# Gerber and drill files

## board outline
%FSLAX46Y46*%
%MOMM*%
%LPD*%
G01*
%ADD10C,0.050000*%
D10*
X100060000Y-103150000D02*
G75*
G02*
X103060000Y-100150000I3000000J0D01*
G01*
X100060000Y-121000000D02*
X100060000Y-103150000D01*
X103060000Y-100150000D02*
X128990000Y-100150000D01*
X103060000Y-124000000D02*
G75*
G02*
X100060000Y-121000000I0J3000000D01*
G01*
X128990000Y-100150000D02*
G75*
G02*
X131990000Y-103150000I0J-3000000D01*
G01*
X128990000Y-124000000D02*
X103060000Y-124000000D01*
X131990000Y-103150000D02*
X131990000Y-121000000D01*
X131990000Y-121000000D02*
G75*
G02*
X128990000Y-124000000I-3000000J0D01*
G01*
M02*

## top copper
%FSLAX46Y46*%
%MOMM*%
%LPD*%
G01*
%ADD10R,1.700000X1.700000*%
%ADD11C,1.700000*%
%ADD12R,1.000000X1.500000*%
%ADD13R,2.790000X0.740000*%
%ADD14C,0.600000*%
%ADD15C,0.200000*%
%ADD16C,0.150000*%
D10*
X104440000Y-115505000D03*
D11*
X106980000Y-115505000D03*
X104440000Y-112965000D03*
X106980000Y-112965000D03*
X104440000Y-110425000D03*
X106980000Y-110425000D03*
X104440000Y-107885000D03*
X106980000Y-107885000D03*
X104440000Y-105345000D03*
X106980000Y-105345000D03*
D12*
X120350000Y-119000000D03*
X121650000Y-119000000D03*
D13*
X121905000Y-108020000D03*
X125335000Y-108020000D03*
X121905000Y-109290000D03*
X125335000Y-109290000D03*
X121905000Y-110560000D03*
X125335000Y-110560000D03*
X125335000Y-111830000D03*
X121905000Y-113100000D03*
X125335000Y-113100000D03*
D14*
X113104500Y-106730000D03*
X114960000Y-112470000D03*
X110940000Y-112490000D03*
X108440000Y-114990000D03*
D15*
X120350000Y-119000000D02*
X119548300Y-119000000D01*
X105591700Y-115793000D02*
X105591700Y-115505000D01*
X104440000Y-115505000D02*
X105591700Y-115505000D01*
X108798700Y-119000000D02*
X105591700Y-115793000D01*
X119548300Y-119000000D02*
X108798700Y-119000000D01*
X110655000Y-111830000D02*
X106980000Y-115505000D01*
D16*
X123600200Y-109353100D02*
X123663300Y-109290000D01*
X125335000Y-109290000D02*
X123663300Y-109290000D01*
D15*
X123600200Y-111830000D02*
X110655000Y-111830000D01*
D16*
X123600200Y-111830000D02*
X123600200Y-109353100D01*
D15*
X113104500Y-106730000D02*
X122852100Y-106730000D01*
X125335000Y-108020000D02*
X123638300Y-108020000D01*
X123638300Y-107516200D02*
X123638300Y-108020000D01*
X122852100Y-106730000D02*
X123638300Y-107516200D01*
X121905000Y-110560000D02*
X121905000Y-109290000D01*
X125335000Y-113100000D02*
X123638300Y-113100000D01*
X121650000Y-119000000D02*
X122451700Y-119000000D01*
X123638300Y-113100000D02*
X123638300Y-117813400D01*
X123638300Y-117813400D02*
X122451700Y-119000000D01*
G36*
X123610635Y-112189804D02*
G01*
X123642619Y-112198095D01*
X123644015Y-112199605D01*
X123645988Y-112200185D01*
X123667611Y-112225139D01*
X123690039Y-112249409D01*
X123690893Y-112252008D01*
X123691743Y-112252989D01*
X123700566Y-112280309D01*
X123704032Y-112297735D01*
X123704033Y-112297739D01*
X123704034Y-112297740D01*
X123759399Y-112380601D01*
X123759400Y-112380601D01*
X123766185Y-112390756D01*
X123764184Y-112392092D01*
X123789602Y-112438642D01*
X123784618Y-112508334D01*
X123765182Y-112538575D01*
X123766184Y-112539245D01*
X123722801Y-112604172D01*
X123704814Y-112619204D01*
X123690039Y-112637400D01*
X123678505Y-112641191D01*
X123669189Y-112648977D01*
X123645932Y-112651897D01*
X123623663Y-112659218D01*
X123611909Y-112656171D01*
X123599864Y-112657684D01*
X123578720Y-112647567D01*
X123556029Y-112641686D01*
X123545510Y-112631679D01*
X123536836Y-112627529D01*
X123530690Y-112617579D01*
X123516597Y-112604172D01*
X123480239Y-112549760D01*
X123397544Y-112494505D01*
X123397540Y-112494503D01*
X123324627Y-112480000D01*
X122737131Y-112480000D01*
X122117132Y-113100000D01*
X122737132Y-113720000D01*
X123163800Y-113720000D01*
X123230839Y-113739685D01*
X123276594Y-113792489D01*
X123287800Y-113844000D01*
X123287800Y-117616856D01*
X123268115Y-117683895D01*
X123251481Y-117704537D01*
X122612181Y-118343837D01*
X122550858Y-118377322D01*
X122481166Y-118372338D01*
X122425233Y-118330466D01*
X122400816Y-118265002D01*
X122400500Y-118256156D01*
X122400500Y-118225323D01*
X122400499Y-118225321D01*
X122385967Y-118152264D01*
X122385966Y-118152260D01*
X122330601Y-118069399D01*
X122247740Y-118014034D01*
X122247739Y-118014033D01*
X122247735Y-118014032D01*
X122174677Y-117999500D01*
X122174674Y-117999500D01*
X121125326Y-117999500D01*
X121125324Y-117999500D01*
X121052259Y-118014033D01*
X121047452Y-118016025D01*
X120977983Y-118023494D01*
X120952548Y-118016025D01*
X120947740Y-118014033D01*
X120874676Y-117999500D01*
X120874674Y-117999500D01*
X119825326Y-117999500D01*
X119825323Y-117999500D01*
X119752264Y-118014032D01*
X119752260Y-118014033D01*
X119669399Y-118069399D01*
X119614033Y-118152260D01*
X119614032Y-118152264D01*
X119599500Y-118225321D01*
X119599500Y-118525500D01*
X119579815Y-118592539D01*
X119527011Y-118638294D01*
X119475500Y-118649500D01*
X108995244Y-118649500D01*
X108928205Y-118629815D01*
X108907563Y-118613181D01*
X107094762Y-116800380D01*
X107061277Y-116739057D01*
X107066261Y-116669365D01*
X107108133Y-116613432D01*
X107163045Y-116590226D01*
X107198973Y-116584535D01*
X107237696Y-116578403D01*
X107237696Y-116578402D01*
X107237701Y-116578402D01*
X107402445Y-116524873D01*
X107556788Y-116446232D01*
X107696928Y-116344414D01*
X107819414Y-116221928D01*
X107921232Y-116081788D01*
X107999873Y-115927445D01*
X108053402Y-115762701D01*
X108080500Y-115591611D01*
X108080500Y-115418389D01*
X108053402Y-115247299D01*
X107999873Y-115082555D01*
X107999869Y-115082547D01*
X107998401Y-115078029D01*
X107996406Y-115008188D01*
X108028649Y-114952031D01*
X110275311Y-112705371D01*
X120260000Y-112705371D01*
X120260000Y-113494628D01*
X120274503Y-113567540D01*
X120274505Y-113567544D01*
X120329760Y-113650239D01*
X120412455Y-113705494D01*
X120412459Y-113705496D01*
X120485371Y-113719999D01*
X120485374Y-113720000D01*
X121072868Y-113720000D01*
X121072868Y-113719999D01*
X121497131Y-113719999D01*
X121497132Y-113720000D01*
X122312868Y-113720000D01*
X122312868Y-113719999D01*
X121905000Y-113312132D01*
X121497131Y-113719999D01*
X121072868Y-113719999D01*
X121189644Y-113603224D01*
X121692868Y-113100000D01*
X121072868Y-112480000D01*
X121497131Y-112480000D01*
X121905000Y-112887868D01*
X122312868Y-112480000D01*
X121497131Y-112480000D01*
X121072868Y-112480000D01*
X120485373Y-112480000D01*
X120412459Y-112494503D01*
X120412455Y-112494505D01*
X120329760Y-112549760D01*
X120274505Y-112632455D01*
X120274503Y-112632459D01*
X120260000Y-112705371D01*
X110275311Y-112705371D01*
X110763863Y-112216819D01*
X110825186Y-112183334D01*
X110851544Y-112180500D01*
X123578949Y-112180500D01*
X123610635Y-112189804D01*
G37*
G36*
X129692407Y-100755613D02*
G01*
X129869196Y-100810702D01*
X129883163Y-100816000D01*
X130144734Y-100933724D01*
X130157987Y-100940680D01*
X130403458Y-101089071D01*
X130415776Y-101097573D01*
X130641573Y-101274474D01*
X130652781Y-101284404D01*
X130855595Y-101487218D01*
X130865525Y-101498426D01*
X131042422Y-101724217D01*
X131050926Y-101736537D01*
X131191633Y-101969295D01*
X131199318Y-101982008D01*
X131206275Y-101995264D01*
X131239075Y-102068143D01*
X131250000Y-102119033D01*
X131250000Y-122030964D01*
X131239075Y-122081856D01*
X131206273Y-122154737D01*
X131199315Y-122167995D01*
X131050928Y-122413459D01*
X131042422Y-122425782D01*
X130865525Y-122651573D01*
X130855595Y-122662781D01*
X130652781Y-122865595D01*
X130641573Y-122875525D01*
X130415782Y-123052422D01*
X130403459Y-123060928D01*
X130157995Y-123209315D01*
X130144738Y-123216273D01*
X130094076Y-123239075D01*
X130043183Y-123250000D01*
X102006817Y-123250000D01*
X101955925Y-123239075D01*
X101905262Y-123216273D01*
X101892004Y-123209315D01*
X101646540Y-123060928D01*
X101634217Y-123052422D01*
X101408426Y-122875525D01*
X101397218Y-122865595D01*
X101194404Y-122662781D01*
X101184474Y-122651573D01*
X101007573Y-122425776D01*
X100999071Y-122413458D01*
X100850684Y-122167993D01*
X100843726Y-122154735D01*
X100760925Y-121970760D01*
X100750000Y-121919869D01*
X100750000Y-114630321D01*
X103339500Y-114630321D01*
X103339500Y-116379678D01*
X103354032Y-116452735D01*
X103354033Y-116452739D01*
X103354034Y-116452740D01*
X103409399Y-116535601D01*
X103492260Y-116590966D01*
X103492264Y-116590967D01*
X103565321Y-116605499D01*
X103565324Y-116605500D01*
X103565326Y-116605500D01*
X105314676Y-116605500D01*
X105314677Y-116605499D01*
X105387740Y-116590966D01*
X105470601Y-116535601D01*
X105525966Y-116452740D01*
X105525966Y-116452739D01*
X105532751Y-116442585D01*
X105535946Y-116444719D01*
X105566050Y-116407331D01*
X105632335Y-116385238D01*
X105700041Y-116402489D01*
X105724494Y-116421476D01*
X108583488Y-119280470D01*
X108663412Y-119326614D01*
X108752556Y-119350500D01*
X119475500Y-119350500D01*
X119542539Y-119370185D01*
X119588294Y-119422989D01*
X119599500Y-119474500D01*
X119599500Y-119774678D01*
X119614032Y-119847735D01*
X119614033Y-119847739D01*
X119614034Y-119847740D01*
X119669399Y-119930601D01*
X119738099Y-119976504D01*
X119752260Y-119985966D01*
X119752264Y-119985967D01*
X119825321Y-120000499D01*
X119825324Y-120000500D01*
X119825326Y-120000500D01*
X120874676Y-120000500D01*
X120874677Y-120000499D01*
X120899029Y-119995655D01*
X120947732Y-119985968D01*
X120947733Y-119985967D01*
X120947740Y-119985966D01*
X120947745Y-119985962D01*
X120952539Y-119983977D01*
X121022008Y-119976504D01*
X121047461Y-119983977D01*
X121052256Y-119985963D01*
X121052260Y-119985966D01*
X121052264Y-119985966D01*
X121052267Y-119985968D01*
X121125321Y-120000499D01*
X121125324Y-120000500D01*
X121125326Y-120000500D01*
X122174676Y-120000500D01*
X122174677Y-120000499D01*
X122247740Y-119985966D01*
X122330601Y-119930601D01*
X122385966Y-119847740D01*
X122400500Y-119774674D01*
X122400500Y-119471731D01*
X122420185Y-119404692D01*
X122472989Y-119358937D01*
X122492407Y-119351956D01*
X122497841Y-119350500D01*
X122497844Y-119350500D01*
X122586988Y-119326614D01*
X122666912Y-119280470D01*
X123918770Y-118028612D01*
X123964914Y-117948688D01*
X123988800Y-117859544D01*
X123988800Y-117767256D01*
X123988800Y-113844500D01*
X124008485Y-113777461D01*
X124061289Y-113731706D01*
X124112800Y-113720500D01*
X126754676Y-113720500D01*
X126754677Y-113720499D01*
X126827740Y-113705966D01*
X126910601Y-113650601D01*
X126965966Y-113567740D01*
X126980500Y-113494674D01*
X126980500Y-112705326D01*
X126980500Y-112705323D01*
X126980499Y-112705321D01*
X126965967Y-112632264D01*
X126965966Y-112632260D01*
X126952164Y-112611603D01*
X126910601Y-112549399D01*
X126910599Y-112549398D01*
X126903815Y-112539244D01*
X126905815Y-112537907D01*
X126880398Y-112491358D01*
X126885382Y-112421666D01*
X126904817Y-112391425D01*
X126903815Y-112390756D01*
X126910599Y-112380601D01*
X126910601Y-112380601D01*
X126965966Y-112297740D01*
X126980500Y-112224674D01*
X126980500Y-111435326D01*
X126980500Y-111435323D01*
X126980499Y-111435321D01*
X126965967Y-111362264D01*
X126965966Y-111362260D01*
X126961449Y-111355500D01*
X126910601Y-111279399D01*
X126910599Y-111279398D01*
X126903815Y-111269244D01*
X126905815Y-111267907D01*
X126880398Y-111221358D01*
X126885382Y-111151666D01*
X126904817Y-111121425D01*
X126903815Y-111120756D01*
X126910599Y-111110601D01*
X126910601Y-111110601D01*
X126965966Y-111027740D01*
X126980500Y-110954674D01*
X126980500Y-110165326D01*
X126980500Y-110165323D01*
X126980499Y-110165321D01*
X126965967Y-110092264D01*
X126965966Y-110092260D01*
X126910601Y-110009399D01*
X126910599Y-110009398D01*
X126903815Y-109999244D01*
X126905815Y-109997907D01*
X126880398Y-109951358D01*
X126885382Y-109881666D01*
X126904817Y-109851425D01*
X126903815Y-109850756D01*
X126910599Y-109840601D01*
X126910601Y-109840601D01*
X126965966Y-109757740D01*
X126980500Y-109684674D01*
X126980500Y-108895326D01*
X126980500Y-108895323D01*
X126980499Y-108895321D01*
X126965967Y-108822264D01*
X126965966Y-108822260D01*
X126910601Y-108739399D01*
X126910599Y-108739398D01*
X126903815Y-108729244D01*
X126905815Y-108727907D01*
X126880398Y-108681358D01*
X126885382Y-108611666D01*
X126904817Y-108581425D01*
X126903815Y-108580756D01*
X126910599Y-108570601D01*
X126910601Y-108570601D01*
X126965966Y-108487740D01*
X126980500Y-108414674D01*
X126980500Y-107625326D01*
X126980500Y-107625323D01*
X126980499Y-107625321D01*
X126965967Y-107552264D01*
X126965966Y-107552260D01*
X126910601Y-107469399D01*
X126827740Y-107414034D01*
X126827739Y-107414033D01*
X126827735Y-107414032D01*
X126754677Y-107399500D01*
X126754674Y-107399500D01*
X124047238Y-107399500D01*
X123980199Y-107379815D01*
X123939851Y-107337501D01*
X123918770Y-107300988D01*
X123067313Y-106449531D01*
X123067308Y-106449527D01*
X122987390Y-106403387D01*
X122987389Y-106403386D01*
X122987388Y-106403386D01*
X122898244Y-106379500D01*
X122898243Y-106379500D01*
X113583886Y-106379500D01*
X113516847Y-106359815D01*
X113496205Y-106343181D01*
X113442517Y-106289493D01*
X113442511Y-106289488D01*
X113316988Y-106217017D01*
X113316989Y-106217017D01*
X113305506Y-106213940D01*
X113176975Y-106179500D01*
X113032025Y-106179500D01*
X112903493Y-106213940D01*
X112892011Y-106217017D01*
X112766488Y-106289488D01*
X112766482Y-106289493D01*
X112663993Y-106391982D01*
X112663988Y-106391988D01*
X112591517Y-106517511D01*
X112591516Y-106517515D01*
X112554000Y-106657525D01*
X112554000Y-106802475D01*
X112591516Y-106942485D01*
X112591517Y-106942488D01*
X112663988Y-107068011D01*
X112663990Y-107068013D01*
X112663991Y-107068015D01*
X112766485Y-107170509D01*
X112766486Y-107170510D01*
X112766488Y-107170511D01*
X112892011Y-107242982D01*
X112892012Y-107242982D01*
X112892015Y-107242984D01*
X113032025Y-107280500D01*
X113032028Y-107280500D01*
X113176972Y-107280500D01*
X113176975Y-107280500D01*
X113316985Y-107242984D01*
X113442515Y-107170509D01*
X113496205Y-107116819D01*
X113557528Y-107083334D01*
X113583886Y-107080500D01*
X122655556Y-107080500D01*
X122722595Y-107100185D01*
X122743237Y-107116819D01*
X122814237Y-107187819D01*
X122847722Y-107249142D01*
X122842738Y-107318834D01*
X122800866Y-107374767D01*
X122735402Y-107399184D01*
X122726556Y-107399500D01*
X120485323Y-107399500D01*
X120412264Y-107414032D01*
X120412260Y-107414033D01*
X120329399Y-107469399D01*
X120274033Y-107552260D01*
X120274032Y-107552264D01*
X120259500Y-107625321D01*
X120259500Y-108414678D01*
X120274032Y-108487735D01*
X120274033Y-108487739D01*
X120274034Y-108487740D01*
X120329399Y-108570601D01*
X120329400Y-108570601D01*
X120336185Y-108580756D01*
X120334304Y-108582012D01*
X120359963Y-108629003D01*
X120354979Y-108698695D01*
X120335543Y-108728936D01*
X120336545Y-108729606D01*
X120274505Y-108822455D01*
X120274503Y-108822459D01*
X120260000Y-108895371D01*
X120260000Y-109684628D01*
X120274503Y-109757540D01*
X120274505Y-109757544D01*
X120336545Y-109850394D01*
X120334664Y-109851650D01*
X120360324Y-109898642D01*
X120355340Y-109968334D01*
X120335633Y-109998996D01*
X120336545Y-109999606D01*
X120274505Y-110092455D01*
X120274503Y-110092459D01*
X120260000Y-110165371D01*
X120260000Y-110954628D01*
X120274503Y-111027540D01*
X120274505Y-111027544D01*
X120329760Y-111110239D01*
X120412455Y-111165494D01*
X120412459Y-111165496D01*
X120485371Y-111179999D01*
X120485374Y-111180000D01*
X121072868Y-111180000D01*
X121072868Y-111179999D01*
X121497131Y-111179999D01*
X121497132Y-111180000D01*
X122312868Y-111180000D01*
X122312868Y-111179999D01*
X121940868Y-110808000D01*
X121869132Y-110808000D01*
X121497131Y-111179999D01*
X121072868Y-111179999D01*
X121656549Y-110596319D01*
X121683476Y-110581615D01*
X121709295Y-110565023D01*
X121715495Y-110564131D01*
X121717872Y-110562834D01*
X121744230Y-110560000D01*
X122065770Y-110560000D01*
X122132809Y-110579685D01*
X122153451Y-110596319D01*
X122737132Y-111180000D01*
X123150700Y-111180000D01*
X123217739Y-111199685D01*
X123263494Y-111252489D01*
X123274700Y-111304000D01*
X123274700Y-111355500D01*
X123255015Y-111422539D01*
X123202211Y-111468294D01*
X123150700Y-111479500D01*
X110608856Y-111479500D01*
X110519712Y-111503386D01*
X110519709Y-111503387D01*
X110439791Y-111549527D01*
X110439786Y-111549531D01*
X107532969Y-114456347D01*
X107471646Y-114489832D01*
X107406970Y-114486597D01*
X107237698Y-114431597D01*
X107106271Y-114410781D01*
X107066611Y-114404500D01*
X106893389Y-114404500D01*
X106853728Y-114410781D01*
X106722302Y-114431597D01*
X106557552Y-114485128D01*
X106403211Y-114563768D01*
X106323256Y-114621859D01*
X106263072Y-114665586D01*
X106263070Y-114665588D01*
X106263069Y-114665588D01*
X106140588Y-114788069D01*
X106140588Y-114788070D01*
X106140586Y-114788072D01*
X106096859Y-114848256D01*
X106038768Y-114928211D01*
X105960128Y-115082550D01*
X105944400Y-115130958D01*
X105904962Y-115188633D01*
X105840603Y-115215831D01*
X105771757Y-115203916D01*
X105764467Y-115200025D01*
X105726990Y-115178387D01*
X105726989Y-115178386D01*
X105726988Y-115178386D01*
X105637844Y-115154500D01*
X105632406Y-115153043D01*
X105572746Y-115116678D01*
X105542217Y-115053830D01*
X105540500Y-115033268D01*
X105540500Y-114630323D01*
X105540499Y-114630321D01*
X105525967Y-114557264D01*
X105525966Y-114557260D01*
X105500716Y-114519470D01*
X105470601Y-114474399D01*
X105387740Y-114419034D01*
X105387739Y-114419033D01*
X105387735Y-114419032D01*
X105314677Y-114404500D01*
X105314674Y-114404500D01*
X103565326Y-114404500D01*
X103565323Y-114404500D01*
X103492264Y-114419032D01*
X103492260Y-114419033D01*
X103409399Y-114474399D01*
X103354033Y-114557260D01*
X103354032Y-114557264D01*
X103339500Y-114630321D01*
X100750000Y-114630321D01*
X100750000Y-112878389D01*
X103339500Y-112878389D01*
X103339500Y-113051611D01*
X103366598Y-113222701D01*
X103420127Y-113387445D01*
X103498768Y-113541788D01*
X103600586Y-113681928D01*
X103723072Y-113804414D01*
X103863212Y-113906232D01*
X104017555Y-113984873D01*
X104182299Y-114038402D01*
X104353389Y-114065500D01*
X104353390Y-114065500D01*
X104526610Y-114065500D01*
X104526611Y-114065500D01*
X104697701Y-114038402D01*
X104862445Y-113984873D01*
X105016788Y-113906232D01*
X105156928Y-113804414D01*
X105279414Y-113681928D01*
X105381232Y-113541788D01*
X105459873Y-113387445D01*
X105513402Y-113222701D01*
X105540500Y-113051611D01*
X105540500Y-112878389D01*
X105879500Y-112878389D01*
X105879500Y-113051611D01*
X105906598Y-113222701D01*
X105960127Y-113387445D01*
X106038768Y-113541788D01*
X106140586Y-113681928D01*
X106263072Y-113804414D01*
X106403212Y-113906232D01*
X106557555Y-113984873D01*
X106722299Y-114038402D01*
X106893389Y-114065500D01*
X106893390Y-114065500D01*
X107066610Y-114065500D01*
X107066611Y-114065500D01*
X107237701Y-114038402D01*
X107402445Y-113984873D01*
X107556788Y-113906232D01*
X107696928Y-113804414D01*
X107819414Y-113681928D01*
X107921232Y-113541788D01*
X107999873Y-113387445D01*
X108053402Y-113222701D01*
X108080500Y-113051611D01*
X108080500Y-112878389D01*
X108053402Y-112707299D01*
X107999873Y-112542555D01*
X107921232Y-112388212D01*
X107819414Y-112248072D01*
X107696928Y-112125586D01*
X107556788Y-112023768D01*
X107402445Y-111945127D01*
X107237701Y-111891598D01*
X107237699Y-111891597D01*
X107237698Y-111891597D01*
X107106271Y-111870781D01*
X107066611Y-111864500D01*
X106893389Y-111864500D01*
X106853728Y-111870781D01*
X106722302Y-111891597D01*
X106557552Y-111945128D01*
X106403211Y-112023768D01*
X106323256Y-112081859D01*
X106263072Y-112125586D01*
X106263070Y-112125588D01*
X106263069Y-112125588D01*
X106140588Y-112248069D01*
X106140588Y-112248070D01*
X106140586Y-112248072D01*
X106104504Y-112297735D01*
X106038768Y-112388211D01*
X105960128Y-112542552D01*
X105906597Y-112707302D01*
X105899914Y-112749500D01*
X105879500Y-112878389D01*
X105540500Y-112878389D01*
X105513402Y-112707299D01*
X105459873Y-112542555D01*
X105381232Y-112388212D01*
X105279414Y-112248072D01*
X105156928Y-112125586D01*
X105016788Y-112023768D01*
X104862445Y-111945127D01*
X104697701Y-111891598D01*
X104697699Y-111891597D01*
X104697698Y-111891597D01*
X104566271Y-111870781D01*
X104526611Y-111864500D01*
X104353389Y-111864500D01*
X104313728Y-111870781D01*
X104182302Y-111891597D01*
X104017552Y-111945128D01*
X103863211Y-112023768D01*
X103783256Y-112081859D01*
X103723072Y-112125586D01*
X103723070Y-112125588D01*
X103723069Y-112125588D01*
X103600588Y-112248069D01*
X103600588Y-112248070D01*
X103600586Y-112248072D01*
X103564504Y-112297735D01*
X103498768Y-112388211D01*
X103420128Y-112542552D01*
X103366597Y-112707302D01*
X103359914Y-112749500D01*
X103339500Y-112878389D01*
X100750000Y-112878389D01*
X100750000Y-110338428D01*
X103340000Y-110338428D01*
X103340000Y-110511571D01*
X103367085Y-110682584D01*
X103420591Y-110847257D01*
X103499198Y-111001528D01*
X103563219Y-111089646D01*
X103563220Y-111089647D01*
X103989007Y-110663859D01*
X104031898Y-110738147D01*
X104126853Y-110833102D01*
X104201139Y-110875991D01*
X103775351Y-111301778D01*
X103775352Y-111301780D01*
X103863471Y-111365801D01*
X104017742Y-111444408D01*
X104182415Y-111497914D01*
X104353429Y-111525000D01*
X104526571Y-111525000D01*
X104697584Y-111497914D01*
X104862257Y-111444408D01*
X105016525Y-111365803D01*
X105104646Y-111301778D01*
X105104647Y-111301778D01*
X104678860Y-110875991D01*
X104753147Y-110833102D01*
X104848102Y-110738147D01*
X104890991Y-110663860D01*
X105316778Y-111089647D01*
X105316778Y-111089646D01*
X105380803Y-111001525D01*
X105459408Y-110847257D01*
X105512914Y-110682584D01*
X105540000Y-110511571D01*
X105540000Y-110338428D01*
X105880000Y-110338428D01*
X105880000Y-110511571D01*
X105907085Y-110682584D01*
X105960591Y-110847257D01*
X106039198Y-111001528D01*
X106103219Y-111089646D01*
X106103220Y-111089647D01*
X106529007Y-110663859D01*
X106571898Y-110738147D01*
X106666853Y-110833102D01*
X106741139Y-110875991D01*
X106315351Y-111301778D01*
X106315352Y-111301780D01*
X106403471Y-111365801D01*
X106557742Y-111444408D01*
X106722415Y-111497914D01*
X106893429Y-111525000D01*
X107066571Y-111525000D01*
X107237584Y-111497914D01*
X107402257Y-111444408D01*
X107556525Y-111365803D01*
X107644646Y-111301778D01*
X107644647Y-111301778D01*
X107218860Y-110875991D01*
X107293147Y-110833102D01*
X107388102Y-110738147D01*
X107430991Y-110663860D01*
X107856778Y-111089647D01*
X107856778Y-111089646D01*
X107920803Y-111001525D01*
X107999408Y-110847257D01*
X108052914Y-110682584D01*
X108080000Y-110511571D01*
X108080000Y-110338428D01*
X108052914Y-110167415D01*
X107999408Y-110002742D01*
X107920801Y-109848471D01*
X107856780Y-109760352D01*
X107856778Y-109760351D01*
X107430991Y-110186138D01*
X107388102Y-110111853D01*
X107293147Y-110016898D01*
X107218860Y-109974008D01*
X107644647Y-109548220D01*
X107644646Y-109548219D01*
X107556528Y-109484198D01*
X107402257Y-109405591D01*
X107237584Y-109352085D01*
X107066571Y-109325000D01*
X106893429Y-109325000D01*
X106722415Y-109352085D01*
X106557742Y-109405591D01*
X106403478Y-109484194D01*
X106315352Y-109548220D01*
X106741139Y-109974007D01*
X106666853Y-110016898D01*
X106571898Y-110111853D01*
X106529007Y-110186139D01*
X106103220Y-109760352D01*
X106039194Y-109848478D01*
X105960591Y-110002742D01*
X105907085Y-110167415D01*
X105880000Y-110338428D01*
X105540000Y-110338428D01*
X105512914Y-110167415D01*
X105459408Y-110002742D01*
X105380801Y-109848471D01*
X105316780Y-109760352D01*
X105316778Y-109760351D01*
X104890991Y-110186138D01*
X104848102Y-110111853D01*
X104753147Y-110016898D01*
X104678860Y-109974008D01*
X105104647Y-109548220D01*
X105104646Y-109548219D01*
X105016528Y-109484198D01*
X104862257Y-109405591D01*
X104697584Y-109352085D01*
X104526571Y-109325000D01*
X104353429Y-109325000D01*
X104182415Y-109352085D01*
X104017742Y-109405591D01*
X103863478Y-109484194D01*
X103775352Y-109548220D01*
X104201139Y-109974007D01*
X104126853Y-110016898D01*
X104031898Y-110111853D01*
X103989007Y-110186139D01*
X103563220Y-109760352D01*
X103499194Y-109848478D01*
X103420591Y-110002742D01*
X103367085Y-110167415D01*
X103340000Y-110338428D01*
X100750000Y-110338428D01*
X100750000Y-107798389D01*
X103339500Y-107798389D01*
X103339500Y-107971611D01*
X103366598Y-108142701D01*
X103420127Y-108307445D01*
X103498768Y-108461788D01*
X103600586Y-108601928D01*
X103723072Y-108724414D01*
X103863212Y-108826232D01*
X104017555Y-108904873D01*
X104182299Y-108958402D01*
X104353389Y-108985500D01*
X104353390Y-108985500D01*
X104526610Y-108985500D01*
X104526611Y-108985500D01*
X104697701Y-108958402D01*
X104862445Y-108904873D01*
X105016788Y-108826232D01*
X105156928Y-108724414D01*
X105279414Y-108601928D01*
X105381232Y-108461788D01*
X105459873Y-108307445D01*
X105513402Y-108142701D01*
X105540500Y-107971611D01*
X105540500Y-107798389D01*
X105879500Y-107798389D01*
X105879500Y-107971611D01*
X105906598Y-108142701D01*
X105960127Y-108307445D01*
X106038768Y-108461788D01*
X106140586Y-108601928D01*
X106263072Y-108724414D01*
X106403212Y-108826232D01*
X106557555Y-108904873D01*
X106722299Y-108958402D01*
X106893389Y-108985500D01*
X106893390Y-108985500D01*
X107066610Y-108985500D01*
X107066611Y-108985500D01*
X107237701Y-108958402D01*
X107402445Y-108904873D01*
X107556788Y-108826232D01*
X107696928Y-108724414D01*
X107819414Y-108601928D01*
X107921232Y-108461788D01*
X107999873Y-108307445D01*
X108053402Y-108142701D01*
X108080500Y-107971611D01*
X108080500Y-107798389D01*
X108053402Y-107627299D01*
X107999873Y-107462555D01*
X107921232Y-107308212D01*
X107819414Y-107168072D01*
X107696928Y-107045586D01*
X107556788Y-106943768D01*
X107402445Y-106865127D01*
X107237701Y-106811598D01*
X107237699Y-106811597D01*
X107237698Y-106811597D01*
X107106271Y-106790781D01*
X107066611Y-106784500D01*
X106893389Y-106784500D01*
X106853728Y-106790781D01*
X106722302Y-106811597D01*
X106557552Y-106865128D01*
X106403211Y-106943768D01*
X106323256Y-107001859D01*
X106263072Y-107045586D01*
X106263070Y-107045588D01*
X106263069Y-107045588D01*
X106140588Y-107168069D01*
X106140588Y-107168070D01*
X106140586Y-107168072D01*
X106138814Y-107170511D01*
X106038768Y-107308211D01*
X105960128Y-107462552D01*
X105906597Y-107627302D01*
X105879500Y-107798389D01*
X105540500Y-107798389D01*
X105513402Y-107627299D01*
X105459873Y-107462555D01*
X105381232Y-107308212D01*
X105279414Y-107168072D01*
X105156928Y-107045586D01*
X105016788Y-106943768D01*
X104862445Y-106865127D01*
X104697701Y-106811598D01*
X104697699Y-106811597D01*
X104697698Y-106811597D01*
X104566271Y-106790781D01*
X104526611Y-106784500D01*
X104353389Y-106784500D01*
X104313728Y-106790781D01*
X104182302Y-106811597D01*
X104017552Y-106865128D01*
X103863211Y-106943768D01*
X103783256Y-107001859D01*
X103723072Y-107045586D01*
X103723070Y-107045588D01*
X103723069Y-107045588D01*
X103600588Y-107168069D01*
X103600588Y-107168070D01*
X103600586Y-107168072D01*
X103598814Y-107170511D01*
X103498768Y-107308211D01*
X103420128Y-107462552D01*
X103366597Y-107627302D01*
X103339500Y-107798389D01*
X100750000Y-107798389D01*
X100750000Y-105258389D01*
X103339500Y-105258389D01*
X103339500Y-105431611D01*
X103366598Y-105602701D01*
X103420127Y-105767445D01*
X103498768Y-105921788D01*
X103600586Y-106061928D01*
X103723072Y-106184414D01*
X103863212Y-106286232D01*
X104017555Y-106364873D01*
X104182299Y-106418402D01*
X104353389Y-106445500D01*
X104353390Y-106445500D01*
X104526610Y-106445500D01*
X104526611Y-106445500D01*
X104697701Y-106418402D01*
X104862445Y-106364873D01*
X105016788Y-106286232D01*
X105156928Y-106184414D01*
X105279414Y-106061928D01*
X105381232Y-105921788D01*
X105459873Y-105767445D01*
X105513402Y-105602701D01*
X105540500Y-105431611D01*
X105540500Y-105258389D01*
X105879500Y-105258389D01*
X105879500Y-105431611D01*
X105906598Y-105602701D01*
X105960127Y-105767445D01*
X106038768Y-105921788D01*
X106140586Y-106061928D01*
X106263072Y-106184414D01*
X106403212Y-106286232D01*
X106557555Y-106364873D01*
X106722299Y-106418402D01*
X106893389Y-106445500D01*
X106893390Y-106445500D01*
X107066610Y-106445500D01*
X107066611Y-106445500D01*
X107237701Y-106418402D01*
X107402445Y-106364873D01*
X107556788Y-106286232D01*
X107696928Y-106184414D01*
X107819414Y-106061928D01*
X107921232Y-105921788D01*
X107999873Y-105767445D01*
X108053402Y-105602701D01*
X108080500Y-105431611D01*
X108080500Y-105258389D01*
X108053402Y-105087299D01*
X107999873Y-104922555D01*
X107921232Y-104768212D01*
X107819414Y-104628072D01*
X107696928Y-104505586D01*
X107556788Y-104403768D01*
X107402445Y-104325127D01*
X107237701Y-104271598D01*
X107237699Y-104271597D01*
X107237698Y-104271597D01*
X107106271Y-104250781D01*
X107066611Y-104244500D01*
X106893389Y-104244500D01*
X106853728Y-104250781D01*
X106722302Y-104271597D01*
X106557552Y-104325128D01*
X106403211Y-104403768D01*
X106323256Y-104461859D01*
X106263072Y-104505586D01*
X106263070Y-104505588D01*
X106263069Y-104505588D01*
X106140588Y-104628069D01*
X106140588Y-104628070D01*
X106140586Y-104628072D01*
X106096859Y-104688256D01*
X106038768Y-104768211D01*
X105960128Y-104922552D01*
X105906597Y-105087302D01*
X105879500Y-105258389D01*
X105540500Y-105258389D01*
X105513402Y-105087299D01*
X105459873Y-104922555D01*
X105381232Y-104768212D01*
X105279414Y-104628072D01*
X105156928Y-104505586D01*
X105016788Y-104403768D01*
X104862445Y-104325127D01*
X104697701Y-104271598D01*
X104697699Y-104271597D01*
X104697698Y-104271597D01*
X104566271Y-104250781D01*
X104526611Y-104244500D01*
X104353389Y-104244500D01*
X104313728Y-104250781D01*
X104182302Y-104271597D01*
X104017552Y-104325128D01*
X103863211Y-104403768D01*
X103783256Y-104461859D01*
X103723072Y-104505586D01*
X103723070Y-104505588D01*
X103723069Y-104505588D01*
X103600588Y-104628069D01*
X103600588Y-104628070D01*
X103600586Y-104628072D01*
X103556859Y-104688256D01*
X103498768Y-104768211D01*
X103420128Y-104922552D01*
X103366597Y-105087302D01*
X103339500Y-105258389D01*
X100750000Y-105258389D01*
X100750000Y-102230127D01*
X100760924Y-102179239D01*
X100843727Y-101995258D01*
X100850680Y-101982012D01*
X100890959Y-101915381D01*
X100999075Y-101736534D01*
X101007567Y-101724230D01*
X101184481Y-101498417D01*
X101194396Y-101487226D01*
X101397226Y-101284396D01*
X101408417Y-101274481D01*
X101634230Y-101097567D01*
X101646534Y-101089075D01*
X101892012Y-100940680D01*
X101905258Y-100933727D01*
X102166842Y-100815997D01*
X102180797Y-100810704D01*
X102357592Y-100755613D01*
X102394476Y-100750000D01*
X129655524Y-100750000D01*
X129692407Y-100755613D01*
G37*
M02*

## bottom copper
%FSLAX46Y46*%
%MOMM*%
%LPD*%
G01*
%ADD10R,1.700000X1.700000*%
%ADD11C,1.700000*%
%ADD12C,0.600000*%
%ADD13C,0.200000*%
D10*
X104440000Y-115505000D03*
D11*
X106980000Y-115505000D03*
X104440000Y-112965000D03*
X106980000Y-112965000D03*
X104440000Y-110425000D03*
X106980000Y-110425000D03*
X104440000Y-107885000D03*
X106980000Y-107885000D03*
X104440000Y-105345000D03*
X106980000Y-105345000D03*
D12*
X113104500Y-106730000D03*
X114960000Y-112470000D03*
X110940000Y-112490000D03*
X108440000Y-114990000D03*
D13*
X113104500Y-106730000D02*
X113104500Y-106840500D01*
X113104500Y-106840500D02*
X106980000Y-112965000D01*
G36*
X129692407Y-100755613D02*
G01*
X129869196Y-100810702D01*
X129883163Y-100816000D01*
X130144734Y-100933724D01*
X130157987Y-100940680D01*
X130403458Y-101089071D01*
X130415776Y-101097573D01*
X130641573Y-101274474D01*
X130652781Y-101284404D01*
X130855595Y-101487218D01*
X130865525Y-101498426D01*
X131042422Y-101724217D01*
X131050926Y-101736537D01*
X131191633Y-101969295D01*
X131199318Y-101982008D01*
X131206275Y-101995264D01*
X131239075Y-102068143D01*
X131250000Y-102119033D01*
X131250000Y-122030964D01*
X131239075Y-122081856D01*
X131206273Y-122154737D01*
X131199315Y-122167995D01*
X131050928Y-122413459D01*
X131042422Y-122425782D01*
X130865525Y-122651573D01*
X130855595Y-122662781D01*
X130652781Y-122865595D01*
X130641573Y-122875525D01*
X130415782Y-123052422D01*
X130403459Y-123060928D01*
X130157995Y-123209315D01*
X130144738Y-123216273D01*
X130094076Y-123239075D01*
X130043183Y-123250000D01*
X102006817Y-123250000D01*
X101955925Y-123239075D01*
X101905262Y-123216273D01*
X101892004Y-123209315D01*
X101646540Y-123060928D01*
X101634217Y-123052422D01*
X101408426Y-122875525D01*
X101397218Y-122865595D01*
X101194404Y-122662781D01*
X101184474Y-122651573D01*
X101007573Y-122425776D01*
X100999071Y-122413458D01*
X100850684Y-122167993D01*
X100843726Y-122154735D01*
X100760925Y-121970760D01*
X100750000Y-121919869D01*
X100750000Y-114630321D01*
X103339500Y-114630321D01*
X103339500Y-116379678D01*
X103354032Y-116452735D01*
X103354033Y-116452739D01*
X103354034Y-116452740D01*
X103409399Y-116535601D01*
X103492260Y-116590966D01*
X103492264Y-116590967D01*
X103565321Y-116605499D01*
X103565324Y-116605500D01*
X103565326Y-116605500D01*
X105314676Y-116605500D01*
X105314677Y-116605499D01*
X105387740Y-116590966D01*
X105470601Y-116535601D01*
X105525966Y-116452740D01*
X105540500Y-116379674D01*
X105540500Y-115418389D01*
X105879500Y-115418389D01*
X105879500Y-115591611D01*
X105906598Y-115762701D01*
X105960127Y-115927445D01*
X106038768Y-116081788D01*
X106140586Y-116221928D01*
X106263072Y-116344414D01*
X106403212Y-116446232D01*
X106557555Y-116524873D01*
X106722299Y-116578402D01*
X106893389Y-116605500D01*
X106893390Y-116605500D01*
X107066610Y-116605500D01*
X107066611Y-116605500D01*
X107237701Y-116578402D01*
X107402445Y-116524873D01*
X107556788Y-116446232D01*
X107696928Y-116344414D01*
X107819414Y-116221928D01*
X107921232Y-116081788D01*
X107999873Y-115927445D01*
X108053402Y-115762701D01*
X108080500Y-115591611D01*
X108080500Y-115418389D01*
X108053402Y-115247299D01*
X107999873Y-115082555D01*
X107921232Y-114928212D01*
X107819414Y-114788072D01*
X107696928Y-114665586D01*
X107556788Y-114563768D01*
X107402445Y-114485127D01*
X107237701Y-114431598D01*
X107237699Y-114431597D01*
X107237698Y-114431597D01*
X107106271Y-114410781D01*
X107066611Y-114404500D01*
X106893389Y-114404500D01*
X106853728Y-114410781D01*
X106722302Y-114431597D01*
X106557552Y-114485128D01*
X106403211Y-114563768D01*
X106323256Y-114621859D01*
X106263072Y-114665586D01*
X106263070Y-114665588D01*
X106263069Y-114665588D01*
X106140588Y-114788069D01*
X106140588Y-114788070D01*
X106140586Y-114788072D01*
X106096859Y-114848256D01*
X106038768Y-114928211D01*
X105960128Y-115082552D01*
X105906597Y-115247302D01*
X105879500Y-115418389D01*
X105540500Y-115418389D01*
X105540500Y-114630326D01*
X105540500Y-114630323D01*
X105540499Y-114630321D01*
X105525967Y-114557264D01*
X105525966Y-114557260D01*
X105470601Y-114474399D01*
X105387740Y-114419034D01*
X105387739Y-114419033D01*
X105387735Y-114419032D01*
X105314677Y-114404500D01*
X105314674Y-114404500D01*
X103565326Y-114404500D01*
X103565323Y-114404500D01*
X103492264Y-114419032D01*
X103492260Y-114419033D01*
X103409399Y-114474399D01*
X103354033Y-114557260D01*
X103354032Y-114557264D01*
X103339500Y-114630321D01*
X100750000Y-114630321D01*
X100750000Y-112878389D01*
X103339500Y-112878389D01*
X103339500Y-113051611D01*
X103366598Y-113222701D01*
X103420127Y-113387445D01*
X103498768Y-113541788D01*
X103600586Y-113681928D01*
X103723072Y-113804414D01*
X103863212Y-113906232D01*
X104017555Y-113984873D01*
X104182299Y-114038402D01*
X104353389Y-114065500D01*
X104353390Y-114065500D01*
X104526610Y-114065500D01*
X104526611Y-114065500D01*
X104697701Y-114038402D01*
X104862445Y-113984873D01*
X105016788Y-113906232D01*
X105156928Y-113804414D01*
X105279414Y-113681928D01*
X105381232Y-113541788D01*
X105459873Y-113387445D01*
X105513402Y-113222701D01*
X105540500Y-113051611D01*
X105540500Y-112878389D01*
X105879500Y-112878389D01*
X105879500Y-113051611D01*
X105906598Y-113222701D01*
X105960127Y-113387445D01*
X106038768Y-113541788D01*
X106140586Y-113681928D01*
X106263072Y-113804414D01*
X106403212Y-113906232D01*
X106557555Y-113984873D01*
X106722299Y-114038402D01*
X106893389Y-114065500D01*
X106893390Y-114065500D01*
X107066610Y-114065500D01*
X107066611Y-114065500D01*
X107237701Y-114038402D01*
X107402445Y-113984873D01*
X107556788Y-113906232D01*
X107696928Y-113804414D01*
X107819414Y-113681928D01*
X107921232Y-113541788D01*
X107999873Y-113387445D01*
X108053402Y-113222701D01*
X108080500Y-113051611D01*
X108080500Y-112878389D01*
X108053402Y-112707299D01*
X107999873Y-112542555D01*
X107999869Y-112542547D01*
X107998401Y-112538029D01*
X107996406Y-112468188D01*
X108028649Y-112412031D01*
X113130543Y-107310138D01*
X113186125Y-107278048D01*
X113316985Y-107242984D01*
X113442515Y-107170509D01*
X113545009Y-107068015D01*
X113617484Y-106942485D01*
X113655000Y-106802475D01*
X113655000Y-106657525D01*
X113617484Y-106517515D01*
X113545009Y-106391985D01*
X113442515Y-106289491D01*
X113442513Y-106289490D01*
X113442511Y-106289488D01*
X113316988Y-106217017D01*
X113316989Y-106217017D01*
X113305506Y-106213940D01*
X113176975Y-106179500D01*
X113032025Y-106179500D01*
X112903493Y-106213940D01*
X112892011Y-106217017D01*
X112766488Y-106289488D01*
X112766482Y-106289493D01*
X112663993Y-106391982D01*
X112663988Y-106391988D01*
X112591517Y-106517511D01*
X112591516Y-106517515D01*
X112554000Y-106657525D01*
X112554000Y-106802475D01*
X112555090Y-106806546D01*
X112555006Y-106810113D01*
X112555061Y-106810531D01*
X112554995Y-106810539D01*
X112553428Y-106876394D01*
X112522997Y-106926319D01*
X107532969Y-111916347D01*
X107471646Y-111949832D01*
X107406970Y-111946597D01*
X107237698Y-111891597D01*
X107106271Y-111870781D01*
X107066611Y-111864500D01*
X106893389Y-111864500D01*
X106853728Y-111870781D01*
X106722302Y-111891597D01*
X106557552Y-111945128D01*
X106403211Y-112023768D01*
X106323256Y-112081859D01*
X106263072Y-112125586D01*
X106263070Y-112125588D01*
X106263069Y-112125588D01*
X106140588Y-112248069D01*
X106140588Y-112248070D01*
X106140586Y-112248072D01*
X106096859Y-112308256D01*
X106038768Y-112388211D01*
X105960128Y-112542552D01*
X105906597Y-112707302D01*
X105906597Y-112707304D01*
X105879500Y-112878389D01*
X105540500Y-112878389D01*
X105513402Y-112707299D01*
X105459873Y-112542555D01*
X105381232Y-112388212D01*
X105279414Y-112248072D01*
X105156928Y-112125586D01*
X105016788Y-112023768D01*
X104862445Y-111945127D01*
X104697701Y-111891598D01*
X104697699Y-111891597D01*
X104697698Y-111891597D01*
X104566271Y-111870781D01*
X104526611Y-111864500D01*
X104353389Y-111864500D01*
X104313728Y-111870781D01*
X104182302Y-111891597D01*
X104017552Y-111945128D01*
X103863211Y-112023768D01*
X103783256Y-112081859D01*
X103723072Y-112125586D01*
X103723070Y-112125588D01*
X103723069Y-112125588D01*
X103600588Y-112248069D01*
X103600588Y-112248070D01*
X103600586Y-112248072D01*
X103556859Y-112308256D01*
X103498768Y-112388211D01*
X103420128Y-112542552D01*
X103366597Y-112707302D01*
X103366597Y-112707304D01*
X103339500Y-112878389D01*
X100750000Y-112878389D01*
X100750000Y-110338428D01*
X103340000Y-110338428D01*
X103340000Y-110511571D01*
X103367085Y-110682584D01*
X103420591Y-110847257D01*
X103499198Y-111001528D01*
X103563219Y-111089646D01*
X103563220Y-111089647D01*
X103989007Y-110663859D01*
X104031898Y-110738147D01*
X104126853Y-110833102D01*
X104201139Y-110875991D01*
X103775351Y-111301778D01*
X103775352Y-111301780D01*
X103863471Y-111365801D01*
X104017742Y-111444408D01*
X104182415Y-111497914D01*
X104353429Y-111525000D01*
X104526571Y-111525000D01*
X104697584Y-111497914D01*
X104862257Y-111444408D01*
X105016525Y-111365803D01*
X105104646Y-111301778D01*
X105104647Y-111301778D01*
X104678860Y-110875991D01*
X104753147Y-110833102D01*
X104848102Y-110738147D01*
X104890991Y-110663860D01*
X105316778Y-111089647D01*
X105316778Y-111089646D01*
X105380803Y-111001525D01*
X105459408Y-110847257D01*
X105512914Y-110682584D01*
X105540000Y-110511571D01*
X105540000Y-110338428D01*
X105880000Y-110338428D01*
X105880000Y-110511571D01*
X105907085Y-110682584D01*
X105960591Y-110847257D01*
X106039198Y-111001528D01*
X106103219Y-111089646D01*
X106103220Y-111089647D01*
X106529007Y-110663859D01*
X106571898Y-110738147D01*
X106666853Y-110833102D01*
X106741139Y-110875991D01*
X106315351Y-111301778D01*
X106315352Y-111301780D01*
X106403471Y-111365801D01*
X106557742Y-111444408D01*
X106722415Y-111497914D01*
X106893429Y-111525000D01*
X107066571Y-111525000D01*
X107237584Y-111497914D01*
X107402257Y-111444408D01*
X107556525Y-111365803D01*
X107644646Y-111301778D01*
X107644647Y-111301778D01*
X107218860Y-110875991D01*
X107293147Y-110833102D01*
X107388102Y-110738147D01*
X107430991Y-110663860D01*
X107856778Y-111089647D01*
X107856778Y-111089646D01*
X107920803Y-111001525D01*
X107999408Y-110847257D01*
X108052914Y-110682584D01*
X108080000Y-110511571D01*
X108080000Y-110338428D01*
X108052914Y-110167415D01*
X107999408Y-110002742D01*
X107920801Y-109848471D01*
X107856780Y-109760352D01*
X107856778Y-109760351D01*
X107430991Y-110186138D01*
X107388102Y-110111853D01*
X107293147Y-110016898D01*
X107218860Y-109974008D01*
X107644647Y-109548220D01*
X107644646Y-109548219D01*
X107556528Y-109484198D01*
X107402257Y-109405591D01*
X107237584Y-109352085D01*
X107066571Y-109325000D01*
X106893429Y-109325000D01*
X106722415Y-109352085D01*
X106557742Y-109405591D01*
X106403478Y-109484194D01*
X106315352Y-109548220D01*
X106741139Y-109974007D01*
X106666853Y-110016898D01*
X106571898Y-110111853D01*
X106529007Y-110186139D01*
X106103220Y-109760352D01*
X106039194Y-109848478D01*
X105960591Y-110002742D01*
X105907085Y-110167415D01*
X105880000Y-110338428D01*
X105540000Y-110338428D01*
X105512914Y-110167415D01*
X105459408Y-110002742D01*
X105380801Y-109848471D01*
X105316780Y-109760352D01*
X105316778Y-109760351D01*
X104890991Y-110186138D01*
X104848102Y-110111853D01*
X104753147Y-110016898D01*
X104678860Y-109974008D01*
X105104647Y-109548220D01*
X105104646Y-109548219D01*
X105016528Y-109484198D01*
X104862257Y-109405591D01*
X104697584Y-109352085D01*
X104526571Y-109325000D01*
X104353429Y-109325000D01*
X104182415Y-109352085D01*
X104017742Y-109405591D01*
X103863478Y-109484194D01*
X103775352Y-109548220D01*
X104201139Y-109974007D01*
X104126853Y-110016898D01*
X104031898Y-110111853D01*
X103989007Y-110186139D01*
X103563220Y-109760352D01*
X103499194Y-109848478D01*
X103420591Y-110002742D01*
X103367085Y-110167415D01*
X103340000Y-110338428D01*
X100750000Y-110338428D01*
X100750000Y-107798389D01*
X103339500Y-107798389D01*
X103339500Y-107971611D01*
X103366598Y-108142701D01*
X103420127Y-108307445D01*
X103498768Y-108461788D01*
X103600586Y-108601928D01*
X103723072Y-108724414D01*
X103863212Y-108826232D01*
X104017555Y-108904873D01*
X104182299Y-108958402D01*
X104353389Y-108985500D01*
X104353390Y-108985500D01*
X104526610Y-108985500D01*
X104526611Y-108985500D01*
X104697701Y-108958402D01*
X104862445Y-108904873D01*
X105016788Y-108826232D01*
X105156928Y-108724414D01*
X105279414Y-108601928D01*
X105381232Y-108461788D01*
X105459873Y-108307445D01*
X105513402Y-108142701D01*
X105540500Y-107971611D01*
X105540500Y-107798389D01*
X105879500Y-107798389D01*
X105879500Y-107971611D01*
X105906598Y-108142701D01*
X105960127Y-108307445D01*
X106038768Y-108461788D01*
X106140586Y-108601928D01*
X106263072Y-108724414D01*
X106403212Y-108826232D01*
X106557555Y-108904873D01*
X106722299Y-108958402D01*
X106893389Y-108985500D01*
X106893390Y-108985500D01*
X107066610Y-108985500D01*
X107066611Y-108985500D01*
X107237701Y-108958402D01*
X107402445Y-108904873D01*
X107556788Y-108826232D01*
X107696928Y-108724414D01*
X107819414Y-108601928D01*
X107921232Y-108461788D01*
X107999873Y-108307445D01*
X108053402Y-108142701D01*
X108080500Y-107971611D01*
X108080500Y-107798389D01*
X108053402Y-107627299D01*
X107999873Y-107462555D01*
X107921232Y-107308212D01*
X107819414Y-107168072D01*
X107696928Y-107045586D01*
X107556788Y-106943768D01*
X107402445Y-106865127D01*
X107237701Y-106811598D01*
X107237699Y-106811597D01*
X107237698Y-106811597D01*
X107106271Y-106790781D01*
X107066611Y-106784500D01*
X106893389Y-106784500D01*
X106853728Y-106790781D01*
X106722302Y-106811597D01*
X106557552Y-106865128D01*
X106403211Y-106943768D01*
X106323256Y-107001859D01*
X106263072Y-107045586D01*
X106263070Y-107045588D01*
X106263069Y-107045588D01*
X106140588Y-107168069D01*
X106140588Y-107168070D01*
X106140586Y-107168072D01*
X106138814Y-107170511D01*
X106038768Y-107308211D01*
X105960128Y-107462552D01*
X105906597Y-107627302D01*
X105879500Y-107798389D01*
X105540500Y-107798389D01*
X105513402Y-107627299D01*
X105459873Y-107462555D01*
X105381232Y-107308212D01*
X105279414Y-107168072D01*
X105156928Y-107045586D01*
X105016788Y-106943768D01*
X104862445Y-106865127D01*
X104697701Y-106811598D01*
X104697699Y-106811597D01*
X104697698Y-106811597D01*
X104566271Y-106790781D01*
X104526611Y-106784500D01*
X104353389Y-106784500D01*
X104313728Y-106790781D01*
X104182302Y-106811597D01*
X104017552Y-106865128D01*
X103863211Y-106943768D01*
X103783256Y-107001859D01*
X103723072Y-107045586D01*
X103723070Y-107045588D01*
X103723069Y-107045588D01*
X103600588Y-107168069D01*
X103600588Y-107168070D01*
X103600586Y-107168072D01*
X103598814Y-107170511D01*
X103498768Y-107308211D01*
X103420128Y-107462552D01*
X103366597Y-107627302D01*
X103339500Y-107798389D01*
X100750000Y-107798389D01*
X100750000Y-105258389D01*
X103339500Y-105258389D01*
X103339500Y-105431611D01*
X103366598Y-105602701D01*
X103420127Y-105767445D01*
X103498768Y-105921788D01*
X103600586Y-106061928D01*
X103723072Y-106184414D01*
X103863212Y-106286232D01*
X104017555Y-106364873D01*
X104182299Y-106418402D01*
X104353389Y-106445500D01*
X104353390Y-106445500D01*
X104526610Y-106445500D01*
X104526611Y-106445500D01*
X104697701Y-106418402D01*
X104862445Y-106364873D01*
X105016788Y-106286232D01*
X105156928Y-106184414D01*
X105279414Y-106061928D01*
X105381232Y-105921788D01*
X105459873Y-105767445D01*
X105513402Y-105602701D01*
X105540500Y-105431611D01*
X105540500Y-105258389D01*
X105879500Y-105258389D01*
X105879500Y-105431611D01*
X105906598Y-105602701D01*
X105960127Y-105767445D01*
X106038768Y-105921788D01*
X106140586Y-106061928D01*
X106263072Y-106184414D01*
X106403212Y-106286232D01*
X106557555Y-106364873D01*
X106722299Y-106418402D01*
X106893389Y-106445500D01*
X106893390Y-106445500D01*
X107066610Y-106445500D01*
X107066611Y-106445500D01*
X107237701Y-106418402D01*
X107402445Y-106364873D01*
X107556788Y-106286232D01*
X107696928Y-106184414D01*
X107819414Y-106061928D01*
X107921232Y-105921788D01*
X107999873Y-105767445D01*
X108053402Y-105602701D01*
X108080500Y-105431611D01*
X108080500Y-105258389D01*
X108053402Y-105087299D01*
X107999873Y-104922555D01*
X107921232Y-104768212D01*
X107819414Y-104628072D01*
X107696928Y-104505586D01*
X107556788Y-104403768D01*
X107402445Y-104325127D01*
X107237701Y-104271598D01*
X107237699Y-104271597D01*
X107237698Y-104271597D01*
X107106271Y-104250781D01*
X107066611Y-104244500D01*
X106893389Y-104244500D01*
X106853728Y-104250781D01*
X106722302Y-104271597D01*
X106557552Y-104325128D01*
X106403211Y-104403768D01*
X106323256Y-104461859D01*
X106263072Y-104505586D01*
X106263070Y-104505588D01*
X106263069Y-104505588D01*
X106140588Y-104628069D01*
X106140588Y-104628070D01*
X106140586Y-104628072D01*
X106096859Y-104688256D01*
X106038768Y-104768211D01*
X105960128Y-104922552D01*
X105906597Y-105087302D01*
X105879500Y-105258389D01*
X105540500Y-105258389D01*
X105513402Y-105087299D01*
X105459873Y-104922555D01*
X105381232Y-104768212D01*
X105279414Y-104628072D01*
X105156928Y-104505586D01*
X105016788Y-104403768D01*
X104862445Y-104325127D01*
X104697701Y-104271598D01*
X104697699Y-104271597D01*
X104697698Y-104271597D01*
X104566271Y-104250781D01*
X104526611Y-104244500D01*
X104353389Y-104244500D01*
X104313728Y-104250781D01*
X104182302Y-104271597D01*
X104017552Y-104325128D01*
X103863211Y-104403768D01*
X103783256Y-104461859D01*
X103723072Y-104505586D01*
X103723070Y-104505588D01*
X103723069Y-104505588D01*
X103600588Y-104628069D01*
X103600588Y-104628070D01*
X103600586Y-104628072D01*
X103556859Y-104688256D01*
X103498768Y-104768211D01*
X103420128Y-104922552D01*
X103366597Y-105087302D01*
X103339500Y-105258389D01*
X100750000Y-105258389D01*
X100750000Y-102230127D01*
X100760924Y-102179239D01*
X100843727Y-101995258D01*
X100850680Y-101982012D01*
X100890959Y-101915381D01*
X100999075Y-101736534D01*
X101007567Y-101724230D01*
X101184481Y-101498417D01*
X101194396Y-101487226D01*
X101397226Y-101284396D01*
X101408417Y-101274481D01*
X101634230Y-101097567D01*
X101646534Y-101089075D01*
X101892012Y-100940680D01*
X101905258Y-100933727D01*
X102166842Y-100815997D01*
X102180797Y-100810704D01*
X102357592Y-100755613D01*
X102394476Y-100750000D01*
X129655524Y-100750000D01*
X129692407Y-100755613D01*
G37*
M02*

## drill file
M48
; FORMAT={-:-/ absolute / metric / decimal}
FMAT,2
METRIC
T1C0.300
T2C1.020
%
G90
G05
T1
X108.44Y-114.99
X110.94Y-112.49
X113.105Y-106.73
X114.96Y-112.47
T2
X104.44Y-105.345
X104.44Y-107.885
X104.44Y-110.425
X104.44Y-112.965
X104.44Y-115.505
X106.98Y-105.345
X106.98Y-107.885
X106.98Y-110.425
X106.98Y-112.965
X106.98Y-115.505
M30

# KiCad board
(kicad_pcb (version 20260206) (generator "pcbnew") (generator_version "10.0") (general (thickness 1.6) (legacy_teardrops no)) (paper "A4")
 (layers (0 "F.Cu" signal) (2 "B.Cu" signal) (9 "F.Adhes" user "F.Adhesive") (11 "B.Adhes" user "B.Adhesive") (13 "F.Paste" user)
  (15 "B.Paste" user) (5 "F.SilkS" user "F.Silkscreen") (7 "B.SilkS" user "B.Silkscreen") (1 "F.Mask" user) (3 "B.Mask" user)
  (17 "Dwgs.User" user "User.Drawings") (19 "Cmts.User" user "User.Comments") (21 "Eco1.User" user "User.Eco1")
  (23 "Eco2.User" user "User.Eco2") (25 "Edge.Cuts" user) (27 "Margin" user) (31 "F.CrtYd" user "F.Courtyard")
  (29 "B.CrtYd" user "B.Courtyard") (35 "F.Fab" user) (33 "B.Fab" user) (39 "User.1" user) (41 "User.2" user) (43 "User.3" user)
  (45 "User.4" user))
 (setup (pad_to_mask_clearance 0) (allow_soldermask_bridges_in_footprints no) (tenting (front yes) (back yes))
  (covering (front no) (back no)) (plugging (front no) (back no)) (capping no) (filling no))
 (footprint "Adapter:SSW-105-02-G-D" (layer "F.Cu") (at 104.44 115.505 180)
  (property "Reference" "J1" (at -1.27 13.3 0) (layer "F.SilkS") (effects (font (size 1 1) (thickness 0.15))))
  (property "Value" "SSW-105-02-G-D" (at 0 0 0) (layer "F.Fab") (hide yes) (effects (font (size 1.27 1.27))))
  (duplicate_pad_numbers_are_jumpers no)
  (pad "1" thru_hole rect (at 0 0 180) (size 1.7 1.7) (drill 1.02) (layers "*.Cu") (remove_unused_layers no) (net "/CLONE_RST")
   (thermal_bridge_angle 45))
  (pad "2" thru_hole circle (at -2.54 0 180) (size 1.7 1.7) (drill 1.02) (layers "*.Cu") (remove_unused_layers no) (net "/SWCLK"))
  (pad "3" thru_hole circle (at 0 2.54 180) (size 1.7 1.7) (drill 1.02) (layers "*.Cu") (remove_unused_layers no)
   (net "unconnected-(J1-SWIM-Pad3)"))
  (pad "4" thru_hole circle (at -2.54 2.54 180) (size 1.7 1.7) (drill 1.02) (layers "*.Cu") (remove_unused_layers no) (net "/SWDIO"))
  (pad "5" thru_hole circle (at 0 5.08 180) (size 1.7 1.7) (drill 1.02) (layers "*.Cu") (remove_unused_layers no) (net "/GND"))
  (pad "6" thru_hole circle (at -2.54 5.08 180) (size 1.7 1.7) (drill 1.02) (layers "*.Cu") (remove_unused_layers no) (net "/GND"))
  (pad "7" thru_hole circle (at 0 7.62 180) (size 1.7 1.7) (drill 1.02) (layers "*.Cu") (remove_unused_layers no)
   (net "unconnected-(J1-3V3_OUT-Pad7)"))
  (pad "8" thru_hole circle (at -2.54 7.62 180) (size 1.7 1.7) (drill 1.02) (layers "*.Cu") (remove_unused_layers no)
   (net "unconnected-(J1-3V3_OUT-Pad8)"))
  (pad "9" thru_hole circle (at 0 10.16 180) (size 1.7 1.7) (drill 1.02) (layers "*.Cu") (remove_unused_layers no)
   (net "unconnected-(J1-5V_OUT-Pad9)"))
  (pad "10" thru_hole circle (at -2.54 10.16 180) (size 1.7 1.7) (drill 1.02) (layers "*.Cu") (remove_unused_layers no)
   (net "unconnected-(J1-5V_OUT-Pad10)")))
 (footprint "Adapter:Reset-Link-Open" (layer "F.Cu") (at 121 119)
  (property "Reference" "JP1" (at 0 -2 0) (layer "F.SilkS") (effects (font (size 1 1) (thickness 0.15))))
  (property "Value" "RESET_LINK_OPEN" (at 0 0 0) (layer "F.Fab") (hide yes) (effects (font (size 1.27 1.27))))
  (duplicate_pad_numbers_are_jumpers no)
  (pad "1" smd rect (at -0.65 0) (size 1 1.5) (layers "F.Cu" "F.Mask") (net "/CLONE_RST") (thermal_bridge_angle 45))
  (pad "2" smd rect (at 0.65 0) (size 1 1.5) (layers "F.Cu" "F.Mask") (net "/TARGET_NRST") (thermal_bridge_angle 45)))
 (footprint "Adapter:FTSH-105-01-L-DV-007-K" (layer "F.Cu") (at 123.62 110.56 -90)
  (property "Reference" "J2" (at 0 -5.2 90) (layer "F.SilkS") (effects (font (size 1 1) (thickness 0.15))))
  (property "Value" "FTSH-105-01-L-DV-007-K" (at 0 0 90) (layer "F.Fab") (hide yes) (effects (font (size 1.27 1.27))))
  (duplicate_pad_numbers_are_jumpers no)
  (pad "1" smd rect (at -2.54 1.715 270) (size 0.74 2.79) (layers "F.Cu" "F.Mask" "F.Paste") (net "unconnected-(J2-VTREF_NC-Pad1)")
   (thermal_bridge_angle 45))
  (pad "2" smd rect (at -2.54 -1.715 270) (size 0.74 2.79) (layers "F.Cu" "F.Mask" "F.Paste") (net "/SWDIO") (thermal_bridge_angle 45))
  (pad "3" smd rect (at -1.27 1.715 270) (size 0.74 2.79) (layers "F.Cu" "F.Mask" "F.Paste") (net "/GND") (thermal_bridge_angle 45))
  (pad "4" smd rect (at -1.27 -1.715 270) (size 0.74 2.79) (layers "F.Cu" "F.Mask" "F.Paste") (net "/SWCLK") (thermal_bridge_angle 45))
  (pad "5" smd rect (at 0 1.715 270) (size 0.74 2.79) (layers "F.Cu" "F.Mask" "F.Paste") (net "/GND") (thermal_bridge_angle 45))
  (pad "6" smd rect (at 0 -1.715 270) (size 0.74 2.79) (layers "F.Cu" "F.Mask" "F.Paste") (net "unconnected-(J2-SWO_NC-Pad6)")
   (thermal_bridge_angle 45))
  (pad "8" smd rect (at 1.27 -1.715 270) (size 0.74 2.79) (layers "F.Cu" "F.Mask" "F.Paste") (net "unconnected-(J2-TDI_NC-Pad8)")
   (thermal_bridge_angle 45))
  (pad "9" smd rect (at 2.54 1.715 270) (size 0.74 2.79) (layers "F.Cu" "F.Mask" "F.Paste") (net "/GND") (thermal_bridge_angle 45))
  (pad "10" smd rect (at 2.54 -1.715 270) (size 0.74 2.79) (layers "F.Cu" "F.Mask" "F.Paste") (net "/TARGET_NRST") (thermal_bridge_angle 45)))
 (gr_arc (start 100.06 103.15) (mid 100.93868 101.02868) (end 103.06 100.15) (stroke (width 0.05) (type default)) (layer "Edge.Cuts"))
 (gr_line (start 100.06 121) (end 100.06 103.15) (stroke (width 0.05) (type default)) (layer "Edge.Cuts"))
 (gr_line (start 103.06 100.15) (end 128.99 100.15) (stroke (width 0.05) (type default)) (layer "Edge.Cuts"))
 (gr_arc (start 103.06 124) (mid 100.93868 123.12132) (end 100.06 121) (stroke (width 0.05) (type default)) (layer "Edge.Cuts"))
 (gr_arc (start 128.99 100.15) (mid 131.11132 101.02868) (end 131.99 103.15) (stroke (width 0.05) (type default)) (layer "Edge.Cuts"))
 (gr_line (start 128.99 124) (end 103.06 124) (stroke (width 0.05) (type default)) (layer "Edge.Cuts"))
 (gr_line (start 131.99 103.15) (end 131.99 121) (stroke (width 0.05) (type default)) (layer "Edge.Cuts"))
 (gr_arc (start 131.99 121) (mid 131.11132 123.12132) (end 128.99 124) (stroke (width 0.05) (type default)) (layer "Edge.Cuts"))
 (segment (start 120.35 119) (end 119.5483 119) (width 0.2) (layer "F.Cu") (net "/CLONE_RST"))
 (segment (start 105.5917 115.793) (end 105.5917 115.505) (width 0.2) (layer "F.Cu") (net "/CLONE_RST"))
 (segment (start 104.44 115.505) (end 105.5917 115.505) (width 0.2) (layer "F.Cu") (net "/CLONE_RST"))
 (segment (start 108.7987 119) (end 105.5917 115.793) (width 0.2) (layer "F.Cu") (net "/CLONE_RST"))
 (segment (start 119.5483 119) (end 108.7987 119) (width 0.2) (layer "F.Cu") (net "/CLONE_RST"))
 (segment (start 110.655 111.83) (end 106.98 115.505) (width 0.2) (layer "F.Cu") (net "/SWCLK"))
 (segment (start 123.6002 109.3531) (end 123.6633 109.29) (width 0.15) (layer "F.Cu") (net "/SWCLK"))
 (segment (start 125.335 109.29) (end 123.6633 109.29) (width 0.15) (layer "F.Cu") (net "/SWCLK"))
 (segment (start 123.6002 111.83) (end 110.655 111.83) (width 0.2) (layer "F.Cu") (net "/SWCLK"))
 (segment (start 123.6002 111.83) (end 123.6002 109.3531) (width 0.15) (layer "F.Cu") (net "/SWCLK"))
 (segment (start 113.1045 106.73) (end 122.8521 106.73) (width 0.2) (layer "F.Cu") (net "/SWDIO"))
 (segment (start 125.335 108.02) (end 123.6383 108.02) (width 0.2) (layer "F.Cu") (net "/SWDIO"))
 (segment (start 123.6383 107.5162) (end 123.6383 108.02) (width 0.2) (layer "F.Cu") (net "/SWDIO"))
 (segment (start 122.8521 106.73) (end 123.6383 107.5162) (width 0.2) (layer "F.Cu") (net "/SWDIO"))
 (via (at 113.1045 106.73) (size 0.6) (drill 0.3) (layers "F.Cu" "B.Cu") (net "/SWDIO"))
 (segment (start 113.1045 106.73) (end 113.1045 106.8405) (width 0.2) (layer "B.Cu") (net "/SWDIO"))
 (segment (start 113.1045 106.8405) (end 106.98 112.965) (width 0.2) (layer "B.Cu") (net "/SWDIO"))
 (segment (start 121.905 110.56) (end 121.905 109.29) (width 0.2) (layer "F.Cu") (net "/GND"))
 (via (at 114.96 112.47) (size 0.6) (drill 0.3) (layers "F.Cu" "B.Cu") (free yes) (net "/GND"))
 (via (at 110.94 112.49) (size 0.6) (drill 0.3) (layers "F.Cu" "B.Cu") (free yes) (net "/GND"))
 (via (at 108.44 114.99) (size 0.6) (drill 0.3) (layers "F.Cu" "B.Cu") (free yes) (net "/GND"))
 (segment (start 125.335 113.1) (end 123.6383 113.1) (width 0.2) (layer "F.Cu") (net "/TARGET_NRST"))
 (segment (start 121.65 119) (end 122.4517 119) (width 0.2) (layer "F.Cu") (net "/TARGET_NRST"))
 (segment (start 123.6383 113.1) (end 123.6383 117.8134) (width 0.2) (layer "F.Cu") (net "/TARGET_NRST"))
 (segment (start 123.6383 117.8134) (end 122.4517 119) (width 0.2) (layer "F.Cu") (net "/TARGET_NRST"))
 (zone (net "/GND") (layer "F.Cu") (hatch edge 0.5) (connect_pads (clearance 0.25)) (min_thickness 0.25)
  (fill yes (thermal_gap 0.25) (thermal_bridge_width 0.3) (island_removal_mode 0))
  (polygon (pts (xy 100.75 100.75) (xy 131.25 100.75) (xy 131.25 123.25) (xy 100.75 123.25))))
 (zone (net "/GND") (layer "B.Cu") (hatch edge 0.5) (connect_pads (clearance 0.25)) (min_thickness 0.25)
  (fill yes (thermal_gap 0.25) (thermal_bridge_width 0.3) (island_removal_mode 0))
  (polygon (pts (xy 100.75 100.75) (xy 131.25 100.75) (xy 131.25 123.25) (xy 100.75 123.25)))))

